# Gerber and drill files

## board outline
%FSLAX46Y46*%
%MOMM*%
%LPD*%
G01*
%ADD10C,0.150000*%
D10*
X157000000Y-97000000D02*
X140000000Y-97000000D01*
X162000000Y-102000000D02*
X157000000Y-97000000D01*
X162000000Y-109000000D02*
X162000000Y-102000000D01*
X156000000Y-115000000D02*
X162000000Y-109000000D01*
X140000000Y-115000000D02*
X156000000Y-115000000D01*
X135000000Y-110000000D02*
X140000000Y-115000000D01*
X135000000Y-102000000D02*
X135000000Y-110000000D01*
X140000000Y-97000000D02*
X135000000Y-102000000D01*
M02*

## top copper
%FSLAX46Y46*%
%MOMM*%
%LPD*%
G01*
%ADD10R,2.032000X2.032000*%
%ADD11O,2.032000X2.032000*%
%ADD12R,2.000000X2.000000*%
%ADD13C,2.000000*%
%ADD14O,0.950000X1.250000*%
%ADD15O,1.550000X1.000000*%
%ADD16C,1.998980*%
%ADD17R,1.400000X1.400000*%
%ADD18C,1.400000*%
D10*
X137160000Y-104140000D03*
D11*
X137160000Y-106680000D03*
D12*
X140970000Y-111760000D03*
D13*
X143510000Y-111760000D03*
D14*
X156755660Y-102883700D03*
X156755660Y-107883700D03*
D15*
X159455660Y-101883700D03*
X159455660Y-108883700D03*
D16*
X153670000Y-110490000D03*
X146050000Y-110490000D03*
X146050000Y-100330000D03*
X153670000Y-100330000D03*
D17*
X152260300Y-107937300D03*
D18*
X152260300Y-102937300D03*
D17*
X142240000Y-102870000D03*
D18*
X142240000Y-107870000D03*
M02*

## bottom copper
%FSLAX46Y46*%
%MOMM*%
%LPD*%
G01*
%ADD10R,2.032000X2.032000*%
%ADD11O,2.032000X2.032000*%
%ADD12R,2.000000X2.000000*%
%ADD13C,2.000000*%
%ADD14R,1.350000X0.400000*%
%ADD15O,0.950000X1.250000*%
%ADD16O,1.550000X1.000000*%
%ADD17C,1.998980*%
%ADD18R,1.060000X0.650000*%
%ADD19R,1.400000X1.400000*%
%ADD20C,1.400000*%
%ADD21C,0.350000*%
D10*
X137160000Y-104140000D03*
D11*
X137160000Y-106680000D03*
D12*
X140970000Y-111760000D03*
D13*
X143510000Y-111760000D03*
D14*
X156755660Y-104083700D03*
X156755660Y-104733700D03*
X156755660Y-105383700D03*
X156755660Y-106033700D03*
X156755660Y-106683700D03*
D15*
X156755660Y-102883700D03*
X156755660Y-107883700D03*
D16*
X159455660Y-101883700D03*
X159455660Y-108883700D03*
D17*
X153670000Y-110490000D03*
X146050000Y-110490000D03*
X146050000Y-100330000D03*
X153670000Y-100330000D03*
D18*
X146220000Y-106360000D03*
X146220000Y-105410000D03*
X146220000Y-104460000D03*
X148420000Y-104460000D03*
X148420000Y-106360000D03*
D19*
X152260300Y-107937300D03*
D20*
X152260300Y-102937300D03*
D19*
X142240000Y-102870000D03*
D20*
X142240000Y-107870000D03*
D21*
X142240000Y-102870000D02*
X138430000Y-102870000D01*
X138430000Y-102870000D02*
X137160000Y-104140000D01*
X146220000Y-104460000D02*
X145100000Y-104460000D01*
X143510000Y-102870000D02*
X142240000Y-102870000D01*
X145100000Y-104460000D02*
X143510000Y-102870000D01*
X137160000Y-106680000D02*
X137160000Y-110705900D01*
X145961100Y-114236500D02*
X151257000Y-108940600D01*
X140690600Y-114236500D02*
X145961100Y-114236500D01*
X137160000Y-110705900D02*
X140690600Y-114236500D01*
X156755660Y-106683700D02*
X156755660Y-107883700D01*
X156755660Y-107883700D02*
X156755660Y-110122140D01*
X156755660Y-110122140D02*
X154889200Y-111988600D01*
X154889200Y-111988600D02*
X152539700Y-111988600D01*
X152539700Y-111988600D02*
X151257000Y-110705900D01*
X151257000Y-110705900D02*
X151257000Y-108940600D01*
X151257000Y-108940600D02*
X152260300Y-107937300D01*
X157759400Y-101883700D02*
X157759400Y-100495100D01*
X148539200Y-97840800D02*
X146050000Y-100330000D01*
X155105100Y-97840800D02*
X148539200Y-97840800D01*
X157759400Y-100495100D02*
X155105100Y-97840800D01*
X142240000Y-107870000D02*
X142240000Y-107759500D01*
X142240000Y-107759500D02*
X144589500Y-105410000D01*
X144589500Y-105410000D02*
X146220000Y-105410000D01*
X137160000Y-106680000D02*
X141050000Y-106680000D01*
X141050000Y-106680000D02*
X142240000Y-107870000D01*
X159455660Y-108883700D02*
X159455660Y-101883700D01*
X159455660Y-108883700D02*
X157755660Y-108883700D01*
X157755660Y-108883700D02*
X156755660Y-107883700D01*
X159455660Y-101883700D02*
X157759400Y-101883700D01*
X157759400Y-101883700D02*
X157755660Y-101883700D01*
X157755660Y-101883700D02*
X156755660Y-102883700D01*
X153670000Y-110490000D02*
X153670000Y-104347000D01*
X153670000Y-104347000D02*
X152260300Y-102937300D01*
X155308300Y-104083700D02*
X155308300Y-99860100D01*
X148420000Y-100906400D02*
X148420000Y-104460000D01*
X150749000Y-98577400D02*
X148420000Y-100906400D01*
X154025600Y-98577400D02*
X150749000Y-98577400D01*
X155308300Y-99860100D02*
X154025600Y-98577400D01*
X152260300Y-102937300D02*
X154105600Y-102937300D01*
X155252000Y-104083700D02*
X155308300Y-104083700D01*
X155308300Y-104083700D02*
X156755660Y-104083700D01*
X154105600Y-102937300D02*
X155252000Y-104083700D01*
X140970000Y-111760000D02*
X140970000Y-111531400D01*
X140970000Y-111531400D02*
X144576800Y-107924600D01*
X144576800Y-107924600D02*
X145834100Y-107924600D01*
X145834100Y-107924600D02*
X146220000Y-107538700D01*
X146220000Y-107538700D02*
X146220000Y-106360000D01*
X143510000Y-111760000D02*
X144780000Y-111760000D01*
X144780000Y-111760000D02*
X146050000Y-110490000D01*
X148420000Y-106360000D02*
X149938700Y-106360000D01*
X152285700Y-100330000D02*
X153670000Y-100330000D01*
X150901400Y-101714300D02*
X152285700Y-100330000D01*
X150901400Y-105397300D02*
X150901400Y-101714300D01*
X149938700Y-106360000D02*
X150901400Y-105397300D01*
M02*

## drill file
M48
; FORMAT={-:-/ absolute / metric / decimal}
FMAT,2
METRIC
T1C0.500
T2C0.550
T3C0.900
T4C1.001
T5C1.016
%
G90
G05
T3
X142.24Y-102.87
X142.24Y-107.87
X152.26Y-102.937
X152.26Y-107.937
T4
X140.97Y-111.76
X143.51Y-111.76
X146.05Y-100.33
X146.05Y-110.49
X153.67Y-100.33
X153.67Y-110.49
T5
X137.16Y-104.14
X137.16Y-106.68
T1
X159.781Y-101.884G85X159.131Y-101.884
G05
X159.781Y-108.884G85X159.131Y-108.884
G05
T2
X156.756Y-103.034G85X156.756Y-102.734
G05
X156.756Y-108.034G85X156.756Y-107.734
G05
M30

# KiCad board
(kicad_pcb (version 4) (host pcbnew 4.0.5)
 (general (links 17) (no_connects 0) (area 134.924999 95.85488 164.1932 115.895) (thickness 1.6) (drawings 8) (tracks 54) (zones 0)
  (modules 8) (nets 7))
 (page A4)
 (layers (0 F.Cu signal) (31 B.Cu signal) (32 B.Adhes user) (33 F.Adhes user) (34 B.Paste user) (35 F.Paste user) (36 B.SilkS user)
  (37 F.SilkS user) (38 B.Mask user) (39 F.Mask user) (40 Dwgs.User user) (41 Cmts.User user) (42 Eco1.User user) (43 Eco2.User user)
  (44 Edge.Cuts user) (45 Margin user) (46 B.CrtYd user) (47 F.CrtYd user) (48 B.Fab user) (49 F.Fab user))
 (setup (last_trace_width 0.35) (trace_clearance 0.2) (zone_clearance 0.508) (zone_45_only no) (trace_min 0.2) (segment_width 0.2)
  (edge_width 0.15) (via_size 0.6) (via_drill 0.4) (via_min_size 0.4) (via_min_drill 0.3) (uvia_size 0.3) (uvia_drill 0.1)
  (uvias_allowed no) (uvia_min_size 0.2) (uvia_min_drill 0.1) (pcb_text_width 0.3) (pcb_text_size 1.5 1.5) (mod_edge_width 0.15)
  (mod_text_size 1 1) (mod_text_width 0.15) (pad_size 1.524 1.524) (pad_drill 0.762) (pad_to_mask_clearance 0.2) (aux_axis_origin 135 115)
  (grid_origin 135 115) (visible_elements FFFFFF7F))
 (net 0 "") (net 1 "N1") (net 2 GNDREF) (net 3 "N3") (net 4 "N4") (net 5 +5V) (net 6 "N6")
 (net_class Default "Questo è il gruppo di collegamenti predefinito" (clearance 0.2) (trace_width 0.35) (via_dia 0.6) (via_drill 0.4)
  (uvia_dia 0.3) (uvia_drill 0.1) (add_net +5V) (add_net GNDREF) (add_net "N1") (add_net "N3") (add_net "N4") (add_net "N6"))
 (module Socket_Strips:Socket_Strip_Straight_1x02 (layer F.Cu) (at 137.16 104.14 270)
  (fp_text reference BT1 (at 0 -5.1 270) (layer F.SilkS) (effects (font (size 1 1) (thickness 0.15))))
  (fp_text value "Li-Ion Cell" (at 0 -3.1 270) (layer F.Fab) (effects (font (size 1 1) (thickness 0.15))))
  (pad 1 thru_hole rect (at 0 0 270) (size 2.032 2.032) (drill 1.016) (layers *.Cu *.Mask) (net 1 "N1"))
  (pad 2 thru_hole oval (at 2.54 0 270) (size 2.032 2.032) (drill 1.016) (layers *.Cu *.Mask) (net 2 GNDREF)))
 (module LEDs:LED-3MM (layer F.Cu) (at 140.97 111.76)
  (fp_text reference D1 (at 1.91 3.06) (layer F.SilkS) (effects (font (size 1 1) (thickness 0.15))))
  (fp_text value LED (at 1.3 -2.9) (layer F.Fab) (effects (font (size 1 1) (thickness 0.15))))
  (pad 1 thru_hole rect (at 0 0 90) (size 2 2) (drill 1.00076) (layers *.Cu *.Mask) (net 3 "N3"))
  (pad 2 thru_hole circle (at 2.54 0) (size 2 2) (drill 1.00076) (layers *.Cu *.Mask) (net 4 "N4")))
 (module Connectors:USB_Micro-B (layer B.Cu) (at 158.3182 105.3846 270)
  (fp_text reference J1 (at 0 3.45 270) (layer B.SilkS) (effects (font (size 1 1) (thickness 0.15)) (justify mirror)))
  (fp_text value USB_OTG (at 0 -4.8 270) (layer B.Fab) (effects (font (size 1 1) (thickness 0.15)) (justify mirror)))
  (pad 1 smd rect (at -1.3009 1.56254 180) (size 1.35 0.4) (layers B.Cu B.Paste B.Mask) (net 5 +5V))
  (pad 2 smd rect (at -0.6509 1.56254 180) (size 1.35 0.4) (layers B.Cu B.Paste B.Mask))
  (pad 3 smd rect (at -0.0009 1.56254 180) (size 1.35 0.4) (layers B.Cu B.Paste B.Mask))
  (pad 4 smd rect (at 0.6491 1.56254 180) (size 1.35 0.4) (layers B.Cu B.Paste B.Mask))
  (pad 5 smd rect (at 1.2991 1.56254 180) (size 1.35 0.4) (layers B.Cu B.Paste B.Mask) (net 2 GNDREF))
  (pad 6 thru_hole oval (at -2.5009 1.56254 180) (size 0.95 1.25) (drill oval 0.55 0.85) (layers *.Cu *.Mask) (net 2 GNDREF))
  (pad 6 thru_hole oval (at 2.4991 1.56254 180) (size 0.95 1.25) (drill oval 0.55 0.85) (layers *.Cu *.Mask) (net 2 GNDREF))
  (pad 6 thru_hole oval (at -3.5009 -1.13746 180) (size 1.55 1) (drill oval 1.15 0.5) (layers *.Cu *.Mask) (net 2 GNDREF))
  (pad 6 thru_hole oval (at 3.4991 -1.13746 180) (size 1.55 1) (drill oval 1.15 0.5) (layers *.Cu *.Mask) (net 2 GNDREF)))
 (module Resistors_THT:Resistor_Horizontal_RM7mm (layer F.Cu) (at 153.67 110.49 180)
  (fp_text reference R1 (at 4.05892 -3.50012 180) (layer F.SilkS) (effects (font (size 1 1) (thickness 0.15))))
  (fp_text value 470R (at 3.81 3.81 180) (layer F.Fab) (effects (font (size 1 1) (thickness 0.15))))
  (pad 1 thru_hole circle (at 0 0 180) (size 1.99898 1.99898) (drill 1.00076) (layers *.Cu *.SilkS *.Mask) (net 5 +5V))
  (pad 2 thru_hole circle (at 7.62 0 180) (size 1.99898 1.99898) (drill 1.00076) (layers *.Cu *.SilkS *.Mask) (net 4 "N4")))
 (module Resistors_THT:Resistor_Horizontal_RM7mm (layer F.Cu) (at 146.05 100.33)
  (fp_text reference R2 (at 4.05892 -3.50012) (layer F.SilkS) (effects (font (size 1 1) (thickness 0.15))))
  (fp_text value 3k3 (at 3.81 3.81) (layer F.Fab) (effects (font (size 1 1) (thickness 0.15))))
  (pad 1 thru_hole circle (at 0 0) (size 1.99898 1.99898) (drill 1.00076) (layers *.Cu *.SilkS *.Mask) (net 2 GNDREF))
  (pad 2 thru_hole circle (at 7.62 0) (size 1.99898 1.99898) (drill 1.00076) (layers *.Cu *.SilkS *.Mask) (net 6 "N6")))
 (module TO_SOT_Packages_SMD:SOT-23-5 (layer B.Cu) (at 147.32 105.41)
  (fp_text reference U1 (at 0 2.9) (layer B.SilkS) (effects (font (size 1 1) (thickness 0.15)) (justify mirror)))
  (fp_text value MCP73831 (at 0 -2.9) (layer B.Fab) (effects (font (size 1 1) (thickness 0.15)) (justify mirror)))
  (pad 1 smd rect (at -1.1 0.95) (size 1.06 0.65) (layers B.Cu B.Paste B.Mask) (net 3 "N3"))
  (pad 2 smd rect (at -1.1 0) (size 1.06 0.65) (layers B.Cu B.Paste B.Mask) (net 2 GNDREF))
  (pad 3 smd rect (at -1.1 -0.95) (size 1.06 0.65) (layers B.Cu B.Paste B.Mask) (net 1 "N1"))
  (pad 4 smd rect (at 1.1 -0.95) (size 1.06 0.65) (layers B.Cu B.Paste B.Mask) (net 5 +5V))
  (pad 5 smd rect (at 1.1 0.95) (size 1.06 0.65) (layers B.Cu B.Paste B.Mask) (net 6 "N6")))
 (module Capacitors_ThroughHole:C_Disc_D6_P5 (layer F.Cu) (at 152.2603 107.9373 90)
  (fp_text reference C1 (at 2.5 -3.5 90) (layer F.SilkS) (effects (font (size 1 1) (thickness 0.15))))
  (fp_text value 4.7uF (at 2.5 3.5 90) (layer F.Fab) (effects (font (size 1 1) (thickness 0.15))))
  (pad 1 thru_hole rect (at 0 0 90) (size 1.4 1.4) (drill 0.9) (layers *.Cu *.Mask) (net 2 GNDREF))
  (pad 2 thru_hole circle (at 5 0 90) (size 1.4 1.4) (drill 0.9) (layers *.Cu *.Mask) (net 5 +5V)))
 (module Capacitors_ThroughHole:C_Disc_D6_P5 (layer F.Cu) (at 142.24 102.87 270)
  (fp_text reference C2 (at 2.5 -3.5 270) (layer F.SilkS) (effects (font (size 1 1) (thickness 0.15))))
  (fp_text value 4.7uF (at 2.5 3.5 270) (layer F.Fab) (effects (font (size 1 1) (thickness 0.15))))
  (pad 1 thru_hole rect (at 0 0 270) (size 1.4 1.4) (drill 0.9) (layers *.Cu *.Mask) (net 1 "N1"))
  (pad 2 thru_hole circle (at 5 0 270) (size 1.4 1.4) (drill 0.9) (layers *.Cu *.Mask) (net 2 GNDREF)))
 (gr_line (start 157 97) (end 140 97) (angle 90) (layer Edge.Cuts) (width 0.15))
 (gr_line (start 162 102) (end 157 97) (angle 90) (layer Edge.Cuts) (width 0.15))
 (gr_line (start 162 109) (end 162 102) (angle 90) (layer Edge.Cuts) (width 0.15))
 (gr_line (start 156 115) (end 162 109) (angle 90) (layer Edge.Cuts) (width 0.15))
 (gr_line (start 140 115) (end 156 115) (angle 90) (layer Edge.Cuts) (width 0.15))
 (gr_line (start 135 110) (end 140 115) (angle 90) (layer Edge.Cuts) (width 0.15))
 (gr_line (start 135 102) (end 135 110) (angle 90) (layer Edge.Cuts) (width 0.15))
 (gr_line (start 140 97) (end 135 102) (angle 90) (layer Edge.Cuts) (width 0.15))
 (segment (start 142.24 102.87) (end 138.43 102.87) (width 0.35) (layer B.Cu) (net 1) (status 400000))
 (segment (start 138.43 102.87) (end 137.16 104.14) (width 0.35) (layer B.Cu) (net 1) (status 800000))
 (segment (start 146.22 104.46) (end 145.1 104.46) (width 0.35) (layer B.Cu) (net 1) (status 400000))
 (segment (start 143.51 102.87) (end 142.24 102.87) (width 0.35) (layer B.Cu) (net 1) (status 800000))
 (segment (start 145.1 104.46) (end 143.51 102.87) (width 0.35) (layer B.Cu) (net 1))
 (segment (start 137.16 106.68) (end 137.16 110.7059) (width 0.35) (layer B.Cu) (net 2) (status 400000))
 (segment (start 145.9611 114.2365) (end 151.257 108.9406) (width 0.35) (layer B.Cu) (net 2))
 (segment (start 140.6906 114.2365) (end 145.9611 114.2365) (width 0.35) (layer B.Cu) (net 2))
 (segment (start 137.16 110.7059) (end 140.6906 114.2365) (width 0.35) (layer B.Cu) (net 2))
 (segment (start 156.75566 106.6837) (end 156.75566 107.8837) (width 0.35) (layer B.Cu) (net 2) (status C00000))
 (segment (start 156.75566 107.8837) (end 156.75566 110.12214) (width 0.35) (layer B.Cu) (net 2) (status 400000))
 (segment (start 156.75566 110.12214) (end 154.8892 111.9886) (width 0.35) (layer B.Cu) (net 2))
 (segment (start 154.8892 111.9886) (end 152.5397 111.9886) (width 0.35) (layer B.Cu) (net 2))
 (segment (start 152.5397 111.9886) (end 151.257 110.7059) (width 0.35) (layer B.Cu) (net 2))
 (segment (start 151.257 110.7059) (end 151.257 108.9406) (width 0.35) (layer B.Cu) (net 2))
 (segment (start 151.257 108.9406) (end 152.2603 107.9373) (width 0.35) (layer B.Cu) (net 2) (status 800000))
 (segment (start 157.7594 101.8837) (end 157.7594 100.4951) (width 0.35) (layer B.Cu) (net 2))
 (segment (start 148.5392 97.8408) (end 146.05 100.33) (width 0.35) (layer B.Cu) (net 2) (status 800000))
 (segment (start 155.1051 97.8408) (end 148.5392 97.8408) (width 0.35) (layer B.Cu) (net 2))
 (segment (start 157.7594 100.4951) (end 155.1051 97.8408) (width 0.35) (layer B.Cu) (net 2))
 (segment (start 142.24 107.87) (end 142.24 107.7595) (width 0.35) (layer B.Cu) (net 2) (status C00000))
 (segment (start 142.24 107.7595) (end 144.5895 105.41) (width 0.35) (layer B.Cu) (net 2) (status 400000))
 (segment (start 144.5895 105.41) (end 146.22 105.41) (width 0.35) (layer B.Cu) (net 2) (status 800000))
 (segment (start 137.16 106.68) (end 141.05 106.68) (width 0.35) (layer B.Cu) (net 2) (status 400000))
 (segment (start 141.05 106.68) (end 142.24 107.87) (width 0.35) (layer B.Cu) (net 2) (status 800000))
 (segment (start 159.45566 108.8837) (end 159.45566 101.8837) (width 0.35) (layer B.Cu) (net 2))
 (segment (start 159.45566 108.8837) (end 157.75566 108.8837) (width 0.35) (layer B.Cu) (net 2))
 (segment (start 157.75566 108.8837) (end 156.75566 107.8837) (width 0.35) (layer B.Cu) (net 2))
 (segment (start 159.45566 101.8837) (end 157.7594 101.8837) (width 0.35) (layer B.Cu) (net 2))
 (segment (start 157.7594 101.8837) (end 157.75566 101.8837) (width 0.35) (layer B.Cu) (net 2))
 (segment (start 157.75566 101.8837) (end 156.75566 102.8837) (width 0.35) (layer B.Cu) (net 2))
 (segment (start 153.67 110.49) (end 153.67 104.347) (width 0.35) (layer B.Cu) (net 5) (status 400000))
 (segment (start 153.67 104.347) (end 152.2603 102.9373) (width 0.35) (layer B.Cu) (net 5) (status 800000))
 (segment (start 155.3083 104.0837) (end 155.3083 99.8601) (width 0.35) (layer B.Cu) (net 5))
 (segment (start 148.42 100.9064) (end 148.42 104.46) (width 0.35) (layer B.Cu) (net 5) (status 800000))
 (segment (start 150.749 98.5774) (end 148.42 100.9064) (width 0.35) (layer B.Cu) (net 5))
 (segment (start 154.0256 98.5774) (end 150.749 98.5774) (width 0.35) (layer B.Cu) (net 5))
 (segment (start 155.3083 99.8601) (end 154.0256 98.5774) (width 0.35) (layer B.Cu) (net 5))
 (segment (start 152.2603 102.9373) (end 154.1056 102.9373) (width 0.35) (layer B.Cu) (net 5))
 (segment (start 155.252 104.0837) (end 155.3083 104.0837) (width 0.35) (layer B.Cu) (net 5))
 (segment (start 155.3083 104.0837) (end 156.75566 104.0837) (width 0.35) (layer B.Cu) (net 5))
 (segment (start 154.1056 102.9373) (end 155.252 104.0837) (width 0.35) (layer B.Cu) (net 5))
 (segment (start 140.97 111.76) (end 140.97 111.5314) (width 0.35) (layer B.Cu) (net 3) (status C00000))
 (segment (start 140.97 111.5314) (end 144.5768 107.9246) (width 0.35) (layer B.Cu) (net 3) (status 400000))
 (segment (start 144.5768 107.9246) (end 145.8341 107.9246) (width 0.35) (layer B.Cu) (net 3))
 (segment (start 145.8341 107.9246) (end 146.22 107.5387) (width 0.35) (layer B.Cu) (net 3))
 (segment (start 146.22 107.5387) (end 146.22 106.36) (width 0.35) (layer B.Cu) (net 3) (status 800000))
 (segment (start 143.51 111.76) (end 144.78 111.76) (width 0.35) (layer B.Cu) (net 4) (status 400000))
 (segment (start 144.78 111.76) (end 146.05 110.49) (width 0.35) (layer B.Cu) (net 4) (status 800000))
 (segment (start 148.42 106.36) (end 149.9387 106.36) (width 0.35) (layer B.Cu) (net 6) (status 400000))
 (segment (start 152.2857 100.33) (end 153.67 100.33) (width 0.35) (layer B.Cu) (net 6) (status 800000))
 (segment (start 150.9014 101.7143) (end 152.2857 100.33) (width 0.35) (layer B.Cu) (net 6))
 (segment (start 150.9014 105.3973) (end 150.9014 101.7143) (width 0.35) (layer B.Cu) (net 6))
 (segment (start 149.9387 106.36) (end 150.9014 105.3973) (width 0.35) (layer B.Cu) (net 6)))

